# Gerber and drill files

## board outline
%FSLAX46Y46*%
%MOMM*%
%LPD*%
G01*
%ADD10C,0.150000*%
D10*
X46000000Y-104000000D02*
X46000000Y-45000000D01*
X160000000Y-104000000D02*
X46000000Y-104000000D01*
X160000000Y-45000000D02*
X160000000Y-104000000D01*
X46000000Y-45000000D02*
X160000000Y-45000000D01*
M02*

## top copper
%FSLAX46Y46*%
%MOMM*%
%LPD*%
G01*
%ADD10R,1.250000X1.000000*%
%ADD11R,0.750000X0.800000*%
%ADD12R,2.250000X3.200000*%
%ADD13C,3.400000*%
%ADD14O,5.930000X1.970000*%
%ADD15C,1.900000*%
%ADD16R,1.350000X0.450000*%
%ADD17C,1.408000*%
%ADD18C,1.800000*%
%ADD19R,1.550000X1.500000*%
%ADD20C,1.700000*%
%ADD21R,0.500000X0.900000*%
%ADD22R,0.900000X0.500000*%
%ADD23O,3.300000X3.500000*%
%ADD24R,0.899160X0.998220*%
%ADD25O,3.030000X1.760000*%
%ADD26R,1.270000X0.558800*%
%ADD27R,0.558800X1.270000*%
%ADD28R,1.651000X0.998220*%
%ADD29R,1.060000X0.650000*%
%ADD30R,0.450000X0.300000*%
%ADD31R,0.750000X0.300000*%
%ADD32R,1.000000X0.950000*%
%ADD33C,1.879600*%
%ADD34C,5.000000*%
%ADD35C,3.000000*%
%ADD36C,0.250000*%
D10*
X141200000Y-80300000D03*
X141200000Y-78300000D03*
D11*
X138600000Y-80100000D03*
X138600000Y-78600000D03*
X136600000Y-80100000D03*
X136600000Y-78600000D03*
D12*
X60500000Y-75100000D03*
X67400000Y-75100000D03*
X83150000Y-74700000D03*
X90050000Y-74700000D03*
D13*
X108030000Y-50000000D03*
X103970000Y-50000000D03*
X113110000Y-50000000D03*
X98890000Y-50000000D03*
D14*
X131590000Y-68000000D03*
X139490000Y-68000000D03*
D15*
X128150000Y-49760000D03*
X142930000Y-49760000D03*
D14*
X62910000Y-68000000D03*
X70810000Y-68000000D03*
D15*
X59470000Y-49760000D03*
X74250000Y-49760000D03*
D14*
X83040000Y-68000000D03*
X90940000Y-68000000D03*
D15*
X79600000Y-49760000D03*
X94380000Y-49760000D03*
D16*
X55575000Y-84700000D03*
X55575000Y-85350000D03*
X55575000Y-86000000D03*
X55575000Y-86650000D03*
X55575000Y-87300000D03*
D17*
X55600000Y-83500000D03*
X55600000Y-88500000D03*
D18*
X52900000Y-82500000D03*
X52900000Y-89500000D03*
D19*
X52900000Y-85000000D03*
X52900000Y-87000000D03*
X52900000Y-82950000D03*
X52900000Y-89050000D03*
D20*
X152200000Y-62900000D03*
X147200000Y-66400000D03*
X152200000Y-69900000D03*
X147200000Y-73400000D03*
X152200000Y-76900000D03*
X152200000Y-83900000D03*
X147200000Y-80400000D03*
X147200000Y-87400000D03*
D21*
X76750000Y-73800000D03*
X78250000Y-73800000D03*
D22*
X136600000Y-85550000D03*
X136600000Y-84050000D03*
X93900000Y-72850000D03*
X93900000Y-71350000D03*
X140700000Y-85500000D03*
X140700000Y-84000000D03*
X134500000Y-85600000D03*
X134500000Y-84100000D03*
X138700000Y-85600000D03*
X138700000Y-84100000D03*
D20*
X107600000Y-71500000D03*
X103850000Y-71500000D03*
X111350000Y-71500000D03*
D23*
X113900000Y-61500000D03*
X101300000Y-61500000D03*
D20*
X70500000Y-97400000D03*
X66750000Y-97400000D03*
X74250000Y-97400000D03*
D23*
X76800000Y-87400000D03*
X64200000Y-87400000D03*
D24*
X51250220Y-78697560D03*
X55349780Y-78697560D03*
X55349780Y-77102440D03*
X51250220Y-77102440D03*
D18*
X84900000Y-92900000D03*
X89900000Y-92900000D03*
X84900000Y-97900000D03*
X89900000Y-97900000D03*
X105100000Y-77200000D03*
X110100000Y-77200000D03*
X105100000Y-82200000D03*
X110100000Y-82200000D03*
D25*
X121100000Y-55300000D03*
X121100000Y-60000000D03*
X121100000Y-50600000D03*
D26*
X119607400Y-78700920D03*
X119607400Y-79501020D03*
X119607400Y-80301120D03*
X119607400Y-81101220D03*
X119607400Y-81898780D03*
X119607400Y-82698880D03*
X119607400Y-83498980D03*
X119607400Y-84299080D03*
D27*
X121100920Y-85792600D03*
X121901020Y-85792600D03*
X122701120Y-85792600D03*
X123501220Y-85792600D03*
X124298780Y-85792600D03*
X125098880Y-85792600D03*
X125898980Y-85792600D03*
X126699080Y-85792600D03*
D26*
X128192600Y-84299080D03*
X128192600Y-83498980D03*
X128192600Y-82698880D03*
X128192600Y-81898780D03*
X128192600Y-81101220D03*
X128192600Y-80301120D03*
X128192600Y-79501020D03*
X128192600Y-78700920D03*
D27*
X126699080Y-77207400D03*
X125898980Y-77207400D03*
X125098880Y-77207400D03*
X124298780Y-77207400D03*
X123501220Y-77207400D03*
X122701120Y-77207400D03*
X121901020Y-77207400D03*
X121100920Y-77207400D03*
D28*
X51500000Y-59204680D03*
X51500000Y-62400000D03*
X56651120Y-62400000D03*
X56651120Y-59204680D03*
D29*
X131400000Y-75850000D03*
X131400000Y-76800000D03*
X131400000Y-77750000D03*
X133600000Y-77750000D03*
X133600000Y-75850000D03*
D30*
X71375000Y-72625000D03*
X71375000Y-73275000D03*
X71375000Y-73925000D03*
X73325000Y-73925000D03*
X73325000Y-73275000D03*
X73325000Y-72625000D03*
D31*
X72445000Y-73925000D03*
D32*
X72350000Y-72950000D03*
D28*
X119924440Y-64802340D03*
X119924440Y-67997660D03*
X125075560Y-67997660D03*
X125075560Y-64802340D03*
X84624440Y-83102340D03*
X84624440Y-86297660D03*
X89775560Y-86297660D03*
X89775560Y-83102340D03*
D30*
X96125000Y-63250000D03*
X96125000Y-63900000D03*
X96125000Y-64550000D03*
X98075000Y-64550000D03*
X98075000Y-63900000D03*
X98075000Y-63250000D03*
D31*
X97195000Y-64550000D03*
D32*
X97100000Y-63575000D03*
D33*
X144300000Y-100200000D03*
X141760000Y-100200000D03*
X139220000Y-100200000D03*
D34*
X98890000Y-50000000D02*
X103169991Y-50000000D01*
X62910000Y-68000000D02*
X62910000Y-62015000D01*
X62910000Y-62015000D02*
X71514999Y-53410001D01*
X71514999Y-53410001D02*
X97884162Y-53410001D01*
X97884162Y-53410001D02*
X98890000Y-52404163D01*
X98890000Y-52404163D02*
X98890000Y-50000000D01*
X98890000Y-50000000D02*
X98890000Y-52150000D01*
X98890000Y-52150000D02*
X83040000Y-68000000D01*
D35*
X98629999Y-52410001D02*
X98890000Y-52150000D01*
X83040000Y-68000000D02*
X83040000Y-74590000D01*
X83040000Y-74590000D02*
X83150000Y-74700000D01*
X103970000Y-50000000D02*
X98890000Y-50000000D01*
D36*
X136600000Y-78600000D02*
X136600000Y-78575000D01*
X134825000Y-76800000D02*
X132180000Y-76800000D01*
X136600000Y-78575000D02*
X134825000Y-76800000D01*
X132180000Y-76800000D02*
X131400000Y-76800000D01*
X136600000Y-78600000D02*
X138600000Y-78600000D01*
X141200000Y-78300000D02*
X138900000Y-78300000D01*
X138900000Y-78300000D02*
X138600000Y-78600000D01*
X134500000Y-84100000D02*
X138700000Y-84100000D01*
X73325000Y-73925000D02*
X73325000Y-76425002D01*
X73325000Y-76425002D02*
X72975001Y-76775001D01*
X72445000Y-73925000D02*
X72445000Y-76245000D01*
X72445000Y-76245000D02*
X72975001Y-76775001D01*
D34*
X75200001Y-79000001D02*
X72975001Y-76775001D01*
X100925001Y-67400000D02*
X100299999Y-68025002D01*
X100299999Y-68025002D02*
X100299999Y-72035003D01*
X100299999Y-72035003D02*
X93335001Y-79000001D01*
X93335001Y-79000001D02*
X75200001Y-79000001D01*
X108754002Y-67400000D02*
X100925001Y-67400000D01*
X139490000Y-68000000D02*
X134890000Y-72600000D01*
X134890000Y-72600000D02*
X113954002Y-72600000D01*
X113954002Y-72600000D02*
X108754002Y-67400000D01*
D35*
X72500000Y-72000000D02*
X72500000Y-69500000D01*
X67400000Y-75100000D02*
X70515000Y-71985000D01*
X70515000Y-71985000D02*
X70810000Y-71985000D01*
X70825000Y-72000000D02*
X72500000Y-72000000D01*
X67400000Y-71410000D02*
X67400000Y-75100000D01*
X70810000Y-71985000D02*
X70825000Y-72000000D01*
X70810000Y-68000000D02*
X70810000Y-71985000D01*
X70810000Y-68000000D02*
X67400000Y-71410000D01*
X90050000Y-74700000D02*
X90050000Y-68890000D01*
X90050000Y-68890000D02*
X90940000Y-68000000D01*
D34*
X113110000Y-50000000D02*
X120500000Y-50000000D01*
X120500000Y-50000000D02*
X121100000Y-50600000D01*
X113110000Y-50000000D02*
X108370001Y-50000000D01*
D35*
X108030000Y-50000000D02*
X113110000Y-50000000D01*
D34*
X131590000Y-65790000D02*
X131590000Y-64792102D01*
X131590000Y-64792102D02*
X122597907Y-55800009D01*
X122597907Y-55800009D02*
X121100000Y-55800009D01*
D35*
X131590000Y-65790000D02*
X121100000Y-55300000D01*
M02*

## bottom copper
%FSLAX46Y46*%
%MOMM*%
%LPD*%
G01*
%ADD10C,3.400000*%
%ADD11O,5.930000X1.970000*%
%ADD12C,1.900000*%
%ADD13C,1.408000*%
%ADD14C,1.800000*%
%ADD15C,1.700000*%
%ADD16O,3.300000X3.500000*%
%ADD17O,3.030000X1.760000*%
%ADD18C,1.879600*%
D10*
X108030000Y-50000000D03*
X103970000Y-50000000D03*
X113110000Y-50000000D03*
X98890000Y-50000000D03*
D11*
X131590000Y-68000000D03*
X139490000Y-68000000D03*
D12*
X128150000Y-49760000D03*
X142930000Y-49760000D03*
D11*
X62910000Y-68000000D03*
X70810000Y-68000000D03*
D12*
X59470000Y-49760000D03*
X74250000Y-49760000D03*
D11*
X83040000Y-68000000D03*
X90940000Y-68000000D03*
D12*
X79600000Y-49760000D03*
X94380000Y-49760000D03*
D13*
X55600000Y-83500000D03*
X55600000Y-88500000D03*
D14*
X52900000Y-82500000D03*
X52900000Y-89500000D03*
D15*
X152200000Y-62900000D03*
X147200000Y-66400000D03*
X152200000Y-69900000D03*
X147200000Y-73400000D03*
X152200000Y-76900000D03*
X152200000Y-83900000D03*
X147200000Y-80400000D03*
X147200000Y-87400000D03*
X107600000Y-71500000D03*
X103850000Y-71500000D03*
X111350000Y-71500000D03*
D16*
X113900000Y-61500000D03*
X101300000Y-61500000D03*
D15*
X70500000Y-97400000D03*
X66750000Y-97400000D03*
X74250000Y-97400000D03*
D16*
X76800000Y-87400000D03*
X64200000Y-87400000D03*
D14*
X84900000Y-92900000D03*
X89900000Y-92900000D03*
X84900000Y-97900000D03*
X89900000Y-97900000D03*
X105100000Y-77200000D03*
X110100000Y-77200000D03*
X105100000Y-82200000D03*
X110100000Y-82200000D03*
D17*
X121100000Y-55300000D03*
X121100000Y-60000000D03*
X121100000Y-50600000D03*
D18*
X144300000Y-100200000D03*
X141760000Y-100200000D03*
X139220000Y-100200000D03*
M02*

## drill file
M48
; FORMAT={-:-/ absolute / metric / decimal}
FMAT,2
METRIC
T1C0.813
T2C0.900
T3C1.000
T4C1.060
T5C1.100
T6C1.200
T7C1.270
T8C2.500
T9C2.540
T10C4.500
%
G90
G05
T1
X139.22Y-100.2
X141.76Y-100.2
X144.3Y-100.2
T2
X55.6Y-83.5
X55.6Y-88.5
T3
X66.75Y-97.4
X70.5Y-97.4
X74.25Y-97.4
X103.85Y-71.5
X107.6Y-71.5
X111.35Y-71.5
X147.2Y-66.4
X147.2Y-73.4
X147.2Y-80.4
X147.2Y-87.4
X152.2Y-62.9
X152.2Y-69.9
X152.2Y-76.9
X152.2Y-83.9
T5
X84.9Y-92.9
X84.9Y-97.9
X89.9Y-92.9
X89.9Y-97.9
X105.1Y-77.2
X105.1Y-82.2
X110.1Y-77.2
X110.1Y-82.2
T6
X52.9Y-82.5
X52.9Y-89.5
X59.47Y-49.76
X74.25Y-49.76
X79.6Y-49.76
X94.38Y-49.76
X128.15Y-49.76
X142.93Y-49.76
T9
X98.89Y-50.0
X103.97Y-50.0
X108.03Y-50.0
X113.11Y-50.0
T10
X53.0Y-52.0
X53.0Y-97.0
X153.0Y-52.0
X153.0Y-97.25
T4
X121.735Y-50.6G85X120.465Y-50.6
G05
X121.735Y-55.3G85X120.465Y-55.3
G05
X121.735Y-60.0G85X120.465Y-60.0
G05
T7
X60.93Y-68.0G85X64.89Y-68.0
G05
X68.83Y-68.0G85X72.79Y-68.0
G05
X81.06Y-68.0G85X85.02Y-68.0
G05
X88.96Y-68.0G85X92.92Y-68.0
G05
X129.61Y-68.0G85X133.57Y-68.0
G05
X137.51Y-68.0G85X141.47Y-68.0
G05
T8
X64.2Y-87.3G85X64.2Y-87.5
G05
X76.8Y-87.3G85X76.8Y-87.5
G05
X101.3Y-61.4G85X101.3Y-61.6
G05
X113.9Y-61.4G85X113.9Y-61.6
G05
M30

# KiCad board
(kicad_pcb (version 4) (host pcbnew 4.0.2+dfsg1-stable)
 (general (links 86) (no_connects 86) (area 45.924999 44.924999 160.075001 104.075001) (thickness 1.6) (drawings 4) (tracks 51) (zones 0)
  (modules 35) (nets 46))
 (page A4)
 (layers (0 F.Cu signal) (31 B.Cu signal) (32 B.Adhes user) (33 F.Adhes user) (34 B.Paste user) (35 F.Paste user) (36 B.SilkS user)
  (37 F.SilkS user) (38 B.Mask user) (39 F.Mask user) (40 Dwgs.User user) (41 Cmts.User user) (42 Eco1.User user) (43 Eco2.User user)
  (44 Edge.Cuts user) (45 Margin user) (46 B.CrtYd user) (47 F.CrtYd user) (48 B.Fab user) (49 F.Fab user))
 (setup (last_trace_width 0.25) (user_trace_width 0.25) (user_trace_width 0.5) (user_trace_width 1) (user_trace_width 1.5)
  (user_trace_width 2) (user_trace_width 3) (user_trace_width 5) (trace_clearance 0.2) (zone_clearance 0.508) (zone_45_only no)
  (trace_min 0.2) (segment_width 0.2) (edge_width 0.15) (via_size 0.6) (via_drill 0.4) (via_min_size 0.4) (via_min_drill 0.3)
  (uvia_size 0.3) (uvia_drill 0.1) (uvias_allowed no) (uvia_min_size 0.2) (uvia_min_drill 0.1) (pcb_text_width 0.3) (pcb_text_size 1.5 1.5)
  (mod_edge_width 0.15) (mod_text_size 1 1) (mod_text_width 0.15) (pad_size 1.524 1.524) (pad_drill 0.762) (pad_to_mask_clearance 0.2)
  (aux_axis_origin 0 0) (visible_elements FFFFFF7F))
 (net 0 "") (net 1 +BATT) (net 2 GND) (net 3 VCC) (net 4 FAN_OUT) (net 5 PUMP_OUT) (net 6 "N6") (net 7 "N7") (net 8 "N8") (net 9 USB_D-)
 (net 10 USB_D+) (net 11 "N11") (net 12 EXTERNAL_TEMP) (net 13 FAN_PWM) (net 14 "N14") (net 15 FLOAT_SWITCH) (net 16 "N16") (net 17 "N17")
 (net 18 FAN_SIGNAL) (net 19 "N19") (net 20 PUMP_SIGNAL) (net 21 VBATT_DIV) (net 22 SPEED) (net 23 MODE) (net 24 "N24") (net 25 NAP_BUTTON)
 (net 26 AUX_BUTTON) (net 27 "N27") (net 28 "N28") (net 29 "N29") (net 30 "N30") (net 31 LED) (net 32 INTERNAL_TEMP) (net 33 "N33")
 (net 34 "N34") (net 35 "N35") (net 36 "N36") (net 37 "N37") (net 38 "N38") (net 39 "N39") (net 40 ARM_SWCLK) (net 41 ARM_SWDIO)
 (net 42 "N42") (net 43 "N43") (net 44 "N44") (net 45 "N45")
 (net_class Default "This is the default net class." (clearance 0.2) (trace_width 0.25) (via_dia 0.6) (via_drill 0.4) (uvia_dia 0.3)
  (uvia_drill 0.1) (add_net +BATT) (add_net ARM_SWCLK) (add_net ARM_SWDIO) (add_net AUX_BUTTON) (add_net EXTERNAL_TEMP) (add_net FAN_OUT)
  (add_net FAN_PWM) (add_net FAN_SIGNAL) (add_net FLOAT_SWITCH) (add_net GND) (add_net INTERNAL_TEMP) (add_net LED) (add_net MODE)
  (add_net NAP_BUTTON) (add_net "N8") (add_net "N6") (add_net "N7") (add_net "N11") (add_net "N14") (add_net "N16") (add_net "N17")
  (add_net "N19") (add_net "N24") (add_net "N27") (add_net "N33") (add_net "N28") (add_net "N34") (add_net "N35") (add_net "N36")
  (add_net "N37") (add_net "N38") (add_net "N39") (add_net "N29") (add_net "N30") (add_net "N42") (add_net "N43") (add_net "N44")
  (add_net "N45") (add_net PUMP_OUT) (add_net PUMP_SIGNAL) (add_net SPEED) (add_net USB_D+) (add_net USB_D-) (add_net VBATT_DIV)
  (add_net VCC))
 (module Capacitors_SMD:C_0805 (layer F.Cu) (at 141.2 79.3 90)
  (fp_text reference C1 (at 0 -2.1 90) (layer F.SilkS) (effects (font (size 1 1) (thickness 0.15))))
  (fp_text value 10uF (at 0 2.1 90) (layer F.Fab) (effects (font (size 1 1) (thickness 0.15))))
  (pad 1 smd rect (at -1 0 90) (size 1 1.25) (layers F.Cu F.Paste F.Mask) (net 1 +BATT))
  (pad 2 smd rect (at 1 0 90) (size 1 1.25) (layers F.Cu F.Paste F.Mask) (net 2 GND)))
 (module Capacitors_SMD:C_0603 (layer F.Cu) (at 138.6 79.35 90)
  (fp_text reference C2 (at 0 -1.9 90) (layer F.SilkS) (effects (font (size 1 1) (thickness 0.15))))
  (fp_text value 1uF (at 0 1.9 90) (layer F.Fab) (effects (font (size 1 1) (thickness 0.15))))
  (pad 1 smd rect (at -0.75 0 90) (size 0.8 0.75) (layers F.Cu F.Paste F.Mask) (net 1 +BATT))
  (pad 2 smd rect (at 0.75 0 90) (size 0.8 0.75) (layers F.Cu F.Paste F.Mask) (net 2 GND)))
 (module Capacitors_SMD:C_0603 (layer F.Cu) (at 136.6 79.35 90)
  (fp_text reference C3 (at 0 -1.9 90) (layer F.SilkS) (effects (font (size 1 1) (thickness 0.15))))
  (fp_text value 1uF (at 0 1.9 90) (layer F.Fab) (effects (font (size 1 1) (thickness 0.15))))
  (pad 1 smd rect (at -0.75 0 90) (size 0.8 0.75) (layers F.Cu F.Paste F.Mask) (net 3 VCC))
  (pad 2 smd rect (at 0.75 0 90) (size 0.8 0.75) (layers F.Cu F.Paste F.Mask) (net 2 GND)))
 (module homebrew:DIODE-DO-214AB (layer F.Cu) (at 63.95 75.1)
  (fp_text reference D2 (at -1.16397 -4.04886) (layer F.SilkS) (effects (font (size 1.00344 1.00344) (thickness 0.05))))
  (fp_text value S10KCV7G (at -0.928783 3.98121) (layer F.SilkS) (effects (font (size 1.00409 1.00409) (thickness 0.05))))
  (pad 1 smd rect (at -3.45 0) (size 2.25 3.2) (layers F.Cu F.Paste F.Mask) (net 1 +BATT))
  (pad 2 smd rect (at 3.45 0) (size 2.25 3.2) (layers F.Cu F.Paste F.Mask) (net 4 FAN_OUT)))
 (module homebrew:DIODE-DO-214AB (layer F.Cu) (at 86.6 74.7)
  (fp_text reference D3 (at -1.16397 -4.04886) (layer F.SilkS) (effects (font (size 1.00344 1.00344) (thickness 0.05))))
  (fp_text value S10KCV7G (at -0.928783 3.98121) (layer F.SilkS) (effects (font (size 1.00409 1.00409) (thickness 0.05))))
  (pad 1 smd rect (at -3.45 0) (size 2.25 3.2) (layers F.Cu F.Paste F.Mask) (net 1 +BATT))
  (pad 2 smd rect (at 3.45 0) (size 2.25 3.2) (layers F.Cu F.Paste F.Mask) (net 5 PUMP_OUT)))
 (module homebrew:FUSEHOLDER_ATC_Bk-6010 (layer F.Cu) (at 106 50 180)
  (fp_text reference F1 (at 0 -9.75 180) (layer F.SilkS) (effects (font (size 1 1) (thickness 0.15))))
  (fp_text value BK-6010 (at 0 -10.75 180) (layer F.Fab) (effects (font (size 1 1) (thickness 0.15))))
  (pad 1 thru_hole circle (at -2.03 0 180) (size 3.4 3.4) (drill 2.54) (layers *.Cu *.Mask) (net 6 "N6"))
  (pad 2 thru_hole circle (at 2.03 0 180) (size 3.4 3.4) (drill 2.54) (layers *.Cu *.Mask) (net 1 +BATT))
  (pad 1 thru_hole circle (at -7.11 0 180) (size 3.4 3.4) (drill 2.54) (layers *.Cu *.Mask) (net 6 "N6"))
  (pad 2 thru_hole circle (at 7.11 0 180) (size 3.4 3.4) (drill 2.54) (layers *.Cu *.Mask) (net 1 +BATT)))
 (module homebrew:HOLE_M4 (layer F.Cu) (at 153 52)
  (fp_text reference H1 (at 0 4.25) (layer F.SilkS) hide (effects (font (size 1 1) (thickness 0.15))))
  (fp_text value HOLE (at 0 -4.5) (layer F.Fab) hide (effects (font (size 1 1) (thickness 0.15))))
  (pad "" np_thru_hole circle (at 0 0) (size 4.5 4.5) (drill 4.5) (layers *.Cu *.Mask) (clearance 2.2)))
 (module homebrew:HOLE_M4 (layer F.Cu) (at 53 52)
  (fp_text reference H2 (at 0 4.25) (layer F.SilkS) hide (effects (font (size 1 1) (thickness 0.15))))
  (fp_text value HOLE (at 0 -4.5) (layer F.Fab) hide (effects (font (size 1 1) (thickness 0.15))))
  (pad "" np_thru_hole circle (at 0 0) (size 4.5 4.5) (drill 4.5) (layers *.Cu *.Mask) (clearance 2.2)))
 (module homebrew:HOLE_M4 (layer F.Cu) (at 53 97)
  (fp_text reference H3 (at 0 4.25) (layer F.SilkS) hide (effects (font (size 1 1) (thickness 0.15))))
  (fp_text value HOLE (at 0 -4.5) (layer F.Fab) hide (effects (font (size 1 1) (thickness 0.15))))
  (pad "" np_thru_hole circle (at 0 0) (size 4.5 4.5) (drill 4.5) (layers *.Cu *.Mask) (clearance 2.2)))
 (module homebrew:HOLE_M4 (layer F.Cu) (at 153 97.25)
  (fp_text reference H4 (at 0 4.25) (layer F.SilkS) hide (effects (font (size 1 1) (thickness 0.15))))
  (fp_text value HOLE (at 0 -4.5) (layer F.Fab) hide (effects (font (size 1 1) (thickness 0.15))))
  (pad "" np_thru_hole circle (at 0 0) (size 4.5 4.5) (drill 4.5) (layers *.Cu *.Mask) (clearance 2.2)))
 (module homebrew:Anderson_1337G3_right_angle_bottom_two (layer F.Cu) (at 135.54 68)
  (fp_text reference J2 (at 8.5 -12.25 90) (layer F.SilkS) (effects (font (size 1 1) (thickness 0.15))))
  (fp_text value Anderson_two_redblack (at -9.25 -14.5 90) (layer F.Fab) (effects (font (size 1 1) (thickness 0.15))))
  (pad 1 thru_hole oval (at -3.95 0) (size 5.93 1.97) (drill oval 5.23 1.27) (layers *.Cu *.Mask) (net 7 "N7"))
  (pad 2 thru_hole oval (at 3.95 0) (size 5.93 1.97) (drill oval 5.23 1.27) (layers *.Cu *.Mask) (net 2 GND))
  (pad "" thru_hole circle (at -7.39 -18.24) (size 1.9 1.9) (drill 1.2) (layers *.Cu *.Mask))
  (pad "" thru_hole circle (at 7.39 -18.24) (size 1.9 1.9) (drill 1.2) (layers *.Cu *.Mask)))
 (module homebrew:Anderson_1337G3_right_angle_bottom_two (layer F.Cu) (at 66.86 68)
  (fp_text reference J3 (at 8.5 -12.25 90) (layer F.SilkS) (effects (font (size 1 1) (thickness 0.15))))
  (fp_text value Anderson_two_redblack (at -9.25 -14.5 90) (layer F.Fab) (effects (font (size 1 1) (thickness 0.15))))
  (pad 1 thru_hole oval (at -3.95 0) (size 5.93 1.97) (drill oval 5.23 1.27) (layers *.Cu *.Mask) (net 1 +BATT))
  (pad 2 thru_hole oval (at 3.95 0) (size 5.93 1.97) (drill oval 5.23 1.27) (layers *.Cu *.Mask) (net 4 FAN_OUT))
  (pad "" thru_hole circle (at -7.39 -18.24) (size 1.9 1.9) (drill 1.2) (layers *.Cu *.Mask))
  (pad "" thru_hole circle (at 7.39 -18.24) (size 1.9 1.9) (drill 1.2) (layers *.Cu *.Mask)))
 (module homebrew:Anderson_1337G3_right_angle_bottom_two (layer F.Cu) (at 86.99 68)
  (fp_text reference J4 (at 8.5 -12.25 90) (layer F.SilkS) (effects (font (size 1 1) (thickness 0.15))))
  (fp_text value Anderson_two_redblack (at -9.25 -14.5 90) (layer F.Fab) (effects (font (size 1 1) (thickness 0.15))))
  (pad 1 thru_hole oval (at -3.95 0) (size 5.93 1.97) (drill oval 5.23 1.27) (layers *.Cu *.Mask) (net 1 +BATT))
  (pad 2 thru_hole oval (at 3.95 0) (size 5.93 1.97) (drill oval 5.23 1.27) (layers *.Cu *.Mask) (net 5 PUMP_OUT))
  (pad "" thru_hole circle (at -7.39 -18.24) (size 1.9 1.9) (drill 1.2) (layers *.Cu *.Mask))
  (pad "" thru_hole circle (at 7.39 -18.24) (size 1.9 1.9) (drill 1.2) (layers *.Cu *.Mask)))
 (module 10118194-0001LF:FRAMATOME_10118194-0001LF (layer F.Cu) (at 52.9 86 270)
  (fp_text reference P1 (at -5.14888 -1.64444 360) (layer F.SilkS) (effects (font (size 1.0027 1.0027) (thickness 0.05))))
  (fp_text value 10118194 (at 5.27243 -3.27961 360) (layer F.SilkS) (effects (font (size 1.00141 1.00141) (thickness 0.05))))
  (pad 1 smd rect (at -1.3 -2.675 90) (size 0.45 1.35) (layers F.Cu F.Paste F.Mask) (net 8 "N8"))
  (pad 2 smd rect (at -0.65 -2.675 90) (size 0.45 1.35) (layers F.Cu F.Paste F.Mask) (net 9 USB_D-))
  (pad 3 smd rect (at 0 -2.675 90) (size 0.45 1.35) (layers F.Cu F.Paste F.Mask) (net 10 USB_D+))
  (pad 4 smd rect (at 0.65 -2.675 90) (size 0.45 1.35) (layers F.Cu F.Paste F.Mask) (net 2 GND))
  (pad 5 smd rect (at 1.3 -2.675 90) (size 0.45 1.35) (layers F.Cu F.Paste F.Mask) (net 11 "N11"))
  (pad P$6 thru_hole circle (at -2.5 -2.7 270) (size 1.408 1.408) (drill 0.9) (layers *.Cu *.Mask F.SilkS))
  (pad P$7 thru_hole circle (at 2.5 -2.7 270) (size 1.408 1.408) (drill 0.9) (layers *.Cu *.Mask F.SilkS))
  (pad P$8 thru_hole circle (at -3.5 0 270) (size 1.8 1.8) (drill 1.2) (layers *.Cu *.Mask F.SilkS))
  (pad P$9 thru_hole circle (at 3.5 0 270) (size 1.8 1.8) (drill 1.2) (layers *.Cu *.Mask F.SilkS))
  (pad P$10 smd rect (at -1 0 270) (size 1.5 1.55) (layers F.Cu F.Paste F.Mask))
  (pad P$11 smd rect (at 1 0 270) (size 1.5 1.55) (layers F.Cu F.Paste F.Mask))
  (pad P$12 smd rect (at -3.05 0 270) (size 1.5 1.55) (layers F.Cu F.Paste F.Mask))
  (pad P$13 smd rect (at 3.05 0 270) (size 1.5 1.55) (layers F.Cu F.Paste F.Mask)))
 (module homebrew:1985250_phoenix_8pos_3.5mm (layer F.Cu) (at 152.2 62.9 90)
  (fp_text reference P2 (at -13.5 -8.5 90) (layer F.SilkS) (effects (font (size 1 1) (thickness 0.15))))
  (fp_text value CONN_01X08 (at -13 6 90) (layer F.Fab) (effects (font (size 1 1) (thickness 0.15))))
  (pad 1 thru_hole circle (at 0 0 90) (size 1.7 1.7) (drill 1) (layers *.Cu *.Mask) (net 3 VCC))
  (pad 2 thru_hole circle (at -3.5 -5 90) (size 1.7 1.7) (drill 1) (layers *.Cu *.Mask) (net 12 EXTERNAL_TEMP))
  (pad 3 thru_hole circle (at -7 0 90) (size 1.7 1.7) (drill 1) (layers *.Cu *.Mask) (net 2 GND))
  (pad 4 thru_hole circle (at -10.5 -5 90) (size 1.7 1.7) (drill 1) (layers *.Cu *.Mask) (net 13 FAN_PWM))
  (pad 5 thru_hole circle (at -14 0 90) (size 1.7 1.7) (drill 1) (layers *.Cu *.Mask) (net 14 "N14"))
  (pad 7 thru_hole circle (at -21 0 90) (size 1.7 1.7) (drill 1) (layers *.Cu *.Mask) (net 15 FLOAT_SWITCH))
  (pad 6 thru_hole circle (at -17.5 -5 90) (size 1.7 1.7) (drill 1) (layers *.Cu *.Mask) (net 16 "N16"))
  (pad 8 thru_hole circle (at -24.5 -5 90) (size 1.7 1.7) (drill 1) (layers *.Cu *.Mask) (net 2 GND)))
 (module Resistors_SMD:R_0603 (layer F.Cu) (at 77.5 73.8)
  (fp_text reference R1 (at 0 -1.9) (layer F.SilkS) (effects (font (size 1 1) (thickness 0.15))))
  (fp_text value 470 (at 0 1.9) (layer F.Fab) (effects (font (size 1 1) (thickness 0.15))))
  (pad 1 smd rect (at -0.75 0) (size 0.5 0.9) (layers F.Cu F.Paste F.Mask) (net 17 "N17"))
  (pad 2 smd rect (at 0.75 0) (size 0.5 0.9) (layers F.Cu F.Paste F.Mask) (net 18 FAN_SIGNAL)))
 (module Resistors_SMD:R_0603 (layer F.Cu) (at 136.6 84.8 90)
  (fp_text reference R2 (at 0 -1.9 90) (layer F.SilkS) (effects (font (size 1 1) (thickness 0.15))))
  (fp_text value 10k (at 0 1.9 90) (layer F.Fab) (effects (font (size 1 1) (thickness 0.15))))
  (pad 1 smd rect (at -0.75 0 90) (size 0.5 0.9) (layers F.Cu F.Paste F.Mask) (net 17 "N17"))
  (pad 2 smd rect (at 0.75 0 90) (size 0.5 0.9) (layers F.Cu F.Paste F.Mask) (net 2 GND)))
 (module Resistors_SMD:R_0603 (layer F.Cu) (at 93.9 72.1 90)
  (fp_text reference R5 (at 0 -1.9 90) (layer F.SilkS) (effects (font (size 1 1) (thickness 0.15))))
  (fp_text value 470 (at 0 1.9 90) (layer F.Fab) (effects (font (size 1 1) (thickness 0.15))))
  (pad 1 smd rect (at -0.75 0 90) (size 0.5 0.9) (layers F.Cu F.Paste F.Mask) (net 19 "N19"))
  (pad 2 smd rect (at 0.75 0 90) (size 0.5 0.9) (layers F.Cu F.Paste F.Mask) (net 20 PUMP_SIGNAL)))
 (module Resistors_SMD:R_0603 (layer F.Cu) (at 140.7 84.75 90)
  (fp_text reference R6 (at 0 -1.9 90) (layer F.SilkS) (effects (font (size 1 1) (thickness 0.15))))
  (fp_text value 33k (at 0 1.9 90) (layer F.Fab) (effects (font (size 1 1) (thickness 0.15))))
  (pad 1 smd rect (at -0.75 0 90) (size 0.5 0.9) (layers F.Cu F.Paste F.Mask) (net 1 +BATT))
  (pad 2 smd rect (at 0.75 0 90) (size 0.5 0.9) (layers F.Cu F.Paste F.Mask) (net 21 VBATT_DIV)))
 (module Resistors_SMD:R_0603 (layer F.Cu) (at 134.5 84.85 90)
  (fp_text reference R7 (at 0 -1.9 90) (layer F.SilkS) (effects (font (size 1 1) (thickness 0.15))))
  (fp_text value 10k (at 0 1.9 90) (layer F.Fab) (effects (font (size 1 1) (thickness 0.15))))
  (pad 1 smd rect (at -0.75 0 90) (size 0.5 0.9) (layers F.Cu F.Paste F.Mask) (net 21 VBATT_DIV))
  (pad 2 smd rect (at 0.75 0 90) (size 0.5 0.9) (layers F.Cu F.Paste F.Mask) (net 2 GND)))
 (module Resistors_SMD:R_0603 (layer F.Cu) (at 138.7 84.85 90)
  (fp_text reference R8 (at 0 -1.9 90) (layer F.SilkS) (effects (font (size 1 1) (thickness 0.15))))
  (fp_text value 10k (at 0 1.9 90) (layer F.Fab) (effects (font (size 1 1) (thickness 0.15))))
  (pad 1 smd rect (at -0.75 0 90) (size 0.5 0.9) (layers F.Cu F.Paste F.Mask) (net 19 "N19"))
  (pad 2 smd rect (at 0.75 0 90) (size 0.5 0.9) (layers F.Cu F.Paste F.Mask) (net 2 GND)))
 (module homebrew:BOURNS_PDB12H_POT (layer F.Cu) (at 107.6 71.5)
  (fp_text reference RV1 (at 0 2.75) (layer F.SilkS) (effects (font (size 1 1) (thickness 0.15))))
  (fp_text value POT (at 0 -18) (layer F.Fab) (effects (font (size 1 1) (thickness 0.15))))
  (pad 2 thru_hole circle (at 0 0) (size 1.7 1.7) (drill 1) (layers *.Cu *.Mask) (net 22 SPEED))
  (pad 1 thru_hole circle (at -3.75 0) (size 1.7 1.7) (drill 1) (layers *.Cu *.Mask) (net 3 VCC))
  (pad 3 thru_hole circle (at 3.75 0) (size 1.7 1.7) (drill 1) (layers *.Cu *.Mask) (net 2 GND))
  (pad "" thru_hole oval (at 6.3 -10) (size 3.3 3.5) (drill oval 2.5 2.7) (layers *.Cu *.Mask))
  (pad "" thru_hole oval (at -6.3 -10) (size 3.3 3.5) (drill oval 2.5 2.7) (layers *.Cu *.Mask)))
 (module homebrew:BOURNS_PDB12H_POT (layer F.Cu) (at 70.5 97.4)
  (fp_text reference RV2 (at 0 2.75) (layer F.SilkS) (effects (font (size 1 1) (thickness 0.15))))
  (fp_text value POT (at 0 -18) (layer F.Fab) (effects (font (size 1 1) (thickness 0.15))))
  (pad 2 thru_hole circle (at 0 0) (size 1.7 1.7) (drill 1) (layers *.Cu *.Mask) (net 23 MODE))
  (pad 1 thru_hole circle (at -3.75 0) (size 1.7 1.7) (drill 1) (layers *.Cu *.Mask) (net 3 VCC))
  (pad 3 thru_hole circle (at 3.75 0) (size 1.7 1.7) (drill 1) (layers *.Cu *.Mask) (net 2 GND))
  (pad "" thru_hole oval (at 6.3 -10) (size 3.3 3.5) (drill oval 2.5 2.7) (layers *.Cu *.Mask))
  (pad "" thru_hole oval (at -6.3 -10) (size 3.3 3.5) (drill oval 2.5 2.7) (layers *.Cu *.Mask)))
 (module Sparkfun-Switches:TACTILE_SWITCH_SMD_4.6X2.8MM (layer F.Cu) (at 53.3 77.9)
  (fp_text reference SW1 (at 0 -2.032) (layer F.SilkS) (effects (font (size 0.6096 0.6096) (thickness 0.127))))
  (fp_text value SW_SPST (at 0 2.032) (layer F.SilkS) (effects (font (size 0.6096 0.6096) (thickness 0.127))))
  (pad 1 smd rect (at -2.04978 0.79756) (size 0.89916 0.99822) (layers F.Cu F.Paste F.Mask) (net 2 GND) (solder_mask_margin 0.1016))
  (pad 2 smd rect (at 2.04978 0.79756) (size 0.89916 0.99822) (layers F.Cu F.Paste F.Mask) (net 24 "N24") (solder_mask_margin 0.1016))
  (pad 3 smd rect (at 2.04978 -0.79756) (size 0.89916 0.99822) (layers F.Cu F.Paste F.Mask) (solder_mask_margin 0.1016))
  (pad 4 smd rect (at -2.04978 -0.79756) (size 0.89916 0.99822) (layers F.Cu F.Paste F.Mask) (solder_mask_margin 0.1016)))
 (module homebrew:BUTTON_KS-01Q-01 (layer F.Cu) (at 84.9 92.9)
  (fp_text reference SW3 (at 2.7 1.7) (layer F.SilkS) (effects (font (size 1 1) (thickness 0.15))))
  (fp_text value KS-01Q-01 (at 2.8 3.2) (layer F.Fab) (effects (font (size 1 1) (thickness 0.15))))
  (pad 1 thru_hole circle (at 0 0) (size 1.8 1.8) (drill 1.1) (layers *.Cu *.Mask F.SilkS) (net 2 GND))
  (pad 2 thru_hole circle (at 5 0) (size 1.8 1.8) (drill 1.1) (layers *.Cu *.Mask F.SilkS) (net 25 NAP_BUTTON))
  (pad 1 thru_hole circle (at 0 5) (size 1.8 1.8) (drill 1.1) (layers *.Cu *.Mask F.SilkS) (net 2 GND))
  (pad 2 thru_hole circle (at 5 5) (size 1.8 1.8) (drill 1.1) (layers *.Cu *.Mask F.SilkS) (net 25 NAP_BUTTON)))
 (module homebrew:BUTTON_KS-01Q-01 (layer F.Cu) (at 105.1 77.2)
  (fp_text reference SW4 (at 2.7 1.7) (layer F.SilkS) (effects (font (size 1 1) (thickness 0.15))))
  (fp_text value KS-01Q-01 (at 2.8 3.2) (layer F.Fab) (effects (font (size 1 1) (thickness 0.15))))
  (pad 1 thru_hole circle (at 0 0) (size 1.8 1.8) (drill 1.1) (layers *.Cu *.Mask F.SilkS) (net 2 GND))
  (pad 2 thru_hole circle (at 5 0) (size 1.8 1.8) (drill 1.1) (layers *.Cu *.Mask F.SilkS) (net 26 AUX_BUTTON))
  (pad 1 thru_hole circle (at 0 5) (size 1.8 1.8) (drill 1.1) (layers *.Cu *.Mask F.SilkS) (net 2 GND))
  (pad 2 thru_hole circle (at 5 5) (size 1.8 1.8) (drill 1.1) (layers *.Cu *.Mask F.SilkS) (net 26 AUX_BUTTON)))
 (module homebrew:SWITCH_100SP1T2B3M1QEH (layer F.Cu) (at 121.1 55.3 270)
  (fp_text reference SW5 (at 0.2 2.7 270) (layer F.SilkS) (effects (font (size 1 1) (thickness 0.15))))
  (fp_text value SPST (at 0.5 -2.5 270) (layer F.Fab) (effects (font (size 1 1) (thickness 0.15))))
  (pad 2 thru_hole oval (at 0 0 270) (size 1.76 3.03) (drill oval 1.06 2.33) (layers *.Cu *.Mask F.SilkS) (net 7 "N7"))
  (pad 3 thru_hole oval (at 4.7 0 270) (size 1.76 3.03) (drill oval 1.06 2.33) (layers *.Cu *.Mask F.SilkS))
  (pad 1 thru_hole oval (at -4.7 0 270) (size 1.76 3.03) (drill oval 1.06 2.33) (layers *.Cu *.Mask F.SilkS) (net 6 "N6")))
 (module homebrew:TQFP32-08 (layer F.Cu) (at 123.9 81.5)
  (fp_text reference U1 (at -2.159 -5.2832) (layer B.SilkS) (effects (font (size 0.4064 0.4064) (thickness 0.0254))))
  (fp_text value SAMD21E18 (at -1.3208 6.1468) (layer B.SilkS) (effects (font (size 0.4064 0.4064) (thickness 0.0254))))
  (pad 1 smd rect (at -4.2926 -2.79908) (size 1.27 0.5588) (layers F.Cu F.Paste F.Mask) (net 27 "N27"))
  (pad 2 smd rect (at -4.2926 -1.99898) (size 1.27 0.5588) (layers F.Cu F.Paste F.Mask) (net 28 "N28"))
  (pad 3 smd rect (at -4.2926 -1.19888) (size 1.27 0.5588) (layers F.Cu F.Paste F.Mask) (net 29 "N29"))
  (pad 4 smd rect (at -4.2926 -0.39878) (size 1.27 0.5588) (layers F.Cu F.Paste F.Mask) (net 21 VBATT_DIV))
  (pad 5 smd rect (at -4.2926 0.39878) (size 1.27 0.5588) (layers F.Cu F.Paste F.Mask) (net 23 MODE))
  (pad 6 smd rect (at -4.2926 1.19888) (size 1.27 0.5588) (layers F.Cu F.Paste F.Mask) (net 22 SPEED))
  (pad 7 smd rect (at -4.2926 1.99898) (size 1.27 0.5588) (layers F.Cu F.Paste F.Mask) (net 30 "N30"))
  (pad 8 smd rect (at -4.2926 2.79908) (size 1.27 0.5588) (layers F.Cu F.Paste F.Mask) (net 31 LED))
  (pad 9 smd rect (at -2.79908 4.2926) (size 0.5588 1.27) (layers F.Cu F.Paste F.Mask) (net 3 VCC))
  (pad 10 smd rect (at -1.99898 4.2926) (size 0.5588 1.27) (layers F.Cu F.Paste F.Mask) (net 2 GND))
  (pad 11 smd rect (at -1.19888 4.2926) (size 0.5588 1.27) (layers F.Cu F.Paste F.Mask) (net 18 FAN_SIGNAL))
  (pad 12 smd rect (at -0.39878 4.2926) (size 0.5588 1.27) (layers F.Cu F.Paste F.Mask) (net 20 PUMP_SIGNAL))
  (pad 13 smd rect (at 0.39878 4.2926) (size 0.5588 1.27) (layers F.Cu F.Paste F.Mask) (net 13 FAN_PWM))
  (pad 14 smd rect (at 1.19888 4.2926) (size 0.5588 1.27) (layers F.Cu F.Paste F.Mask) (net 25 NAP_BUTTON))
  (pad 15 smd rect (at 1.99898 4.2926) (size 0.5588 1.27) (layers F.Cu F.Paste F.Mask) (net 26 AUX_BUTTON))
  (pad 16 smd rect (at 2.79908 4.2926) (size 0.5588 1.27) (layers F.Cu F.Paste F.Mask) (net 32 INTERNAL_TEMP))
  (pad 17 smd rect (at 4.2926 2.79908) (size 1.27 0.5588) (layers F.Cu F.Paste F.Mask) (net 12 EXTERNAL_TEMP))
  (pad 18 smd rect (at 4.2926 1.99898) (size 1.27 0.5588) (layers F.Cu F.Paste F.Mask) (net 15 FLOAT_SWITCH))
  (pad 19 smd rect (at 4.2926 1.19888) (size 1.27 0.5588) (layers F.Cu F.Paste F.Mask) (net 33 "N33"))
  (pad 20 smd rect (at 4.2926 0.39878) (size 1.27 0.5588) (layers F.Cu F.Paste F.Mask) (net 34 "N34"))
  (pad 21 smd rect (at 4.2926 -0.39878) (size 1.27 0.5588) (layers F.Cu F.Paste F.Mask) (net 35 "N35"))
  (pad 22 smd rect (at 4.2926 -1.19888) (size 1.27 0.5588) (layers F.Cu F.Paste F.Mask) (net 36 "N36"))
  (pad 23 smd rect (at 4.2926 -1.99898) (size 1.27 0.5588) (layers F.Cu F.Paste F.Mask) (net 9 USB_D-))
  (pad 24 smd rect (at 4.2926 -2.79908) (size 1.27 0.5588) (layers F.Cu F.Paste F.Mask) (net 10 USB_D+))
  (pad 25 smd rect (at 2.79908 -4.2926) (size 0.5588 1.27) (layers F.Cu F.Paste F.Mask) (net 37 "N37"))
  (pad 26 smd rect (at 1.99898 -4.2926) (size 0.5588 1.27) (layers F.Cu F.Paste F.Mask) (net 24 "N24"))
  (pad 27 smd rect (at 1.19888 -4.2926) (size 0.5588 1.27) (layers F.Cu F.Paste F.Mask) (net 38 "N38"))
  (pad 28 smd rect (at 0.39878 -4.2926) (size 0.5588 1.27) (layers F.Cu F.Paste F.Mask) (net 2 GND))
  (pad 29 smd rect (at -0.39878 -4.2926) (size 0.5588 1.27) (layers F.Cu F.Paste F.Mask) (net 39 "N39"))
  (pad 30 smd rect (at -1.19888 -4.2926) (size 0.5588 1.27) (layers F.Cu F.Paste F.Mask) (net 3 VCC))
  (pad 31 smd rect (at -1.99898 -4.2926) (size 0.5588 1.27) (layers F.Cu F.Paste F.Mask) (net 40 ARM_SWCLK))
  (pad 32 smd rect (at -2.79908 -4.2926) (size 0.5588 1.27) (layers F.Cu F.Paste F.Mask) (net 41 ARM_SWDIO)))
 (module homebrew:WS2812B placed (layer F.Cu) (at 54.07556 60.80234)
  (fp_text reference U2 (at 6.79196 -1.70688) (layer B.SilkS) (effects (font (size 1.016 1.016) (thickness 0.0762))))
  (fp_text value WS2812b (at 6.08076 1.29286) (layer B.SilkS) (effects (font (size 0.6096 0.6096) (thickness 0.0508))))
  (pad 1 smd rect (at -2.57556 -1.59766) (size 1.651 0.99822) (layers F.Cu F.Paste F.Mask) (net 3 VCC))
  (pad 2 smd rect (at -2.57556 1.59766) (size 1.651 0.99822) (layers F.Cu F.Paste F.Mask) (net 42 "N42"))
  (pad 3 smd rect (at 2.57556 1.59766) (size 1.651 0.99822) (layers F.Cu F.Paste F.Mask) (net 2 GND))
  (pad 4 smd rect (at 2.57556 -1.59766) (size 1.651 0.99822) (layers F.Cu F.Paste F.Mask) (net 31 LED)))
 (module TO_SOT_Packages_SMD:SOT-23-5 (layer F.Cu) (at 132.5 76.8)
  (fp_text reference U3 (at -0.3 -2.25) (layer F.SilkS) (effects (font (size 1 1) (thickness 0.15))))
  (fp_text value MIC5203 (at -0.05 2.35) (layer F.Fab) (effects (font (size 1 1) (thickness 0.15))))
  (pad 1 smd rect (at -1.1 -0.95) (size 1.06 0.65) (layers F.Cu F.Paste F.Mask) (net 1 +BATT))
  (pad 2 smd rect (at -1.1 0) (size 1.06 0.65) (layers F.Cu F.Paste F.Mask) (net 2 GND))
  (pad 3 smd rect (at -1.1 0.95) (size 1.06 0.65) (layers F.Cu F.Paste F.Mask) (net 1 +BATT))
  (pad 4 smd rect (at 1.1 0.95) (size 1.06 0.65) (layers F.Cu F.Paste F.Mask) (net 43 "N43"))
  (pad 5 smd rect (at 1.1 -0.95) (size 1.06 0.65) (layers F.Cu F.Paste F.Mask) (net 3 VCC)))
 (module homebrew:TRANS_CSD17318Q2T (layer F.Cu) (at 72.35 73.275)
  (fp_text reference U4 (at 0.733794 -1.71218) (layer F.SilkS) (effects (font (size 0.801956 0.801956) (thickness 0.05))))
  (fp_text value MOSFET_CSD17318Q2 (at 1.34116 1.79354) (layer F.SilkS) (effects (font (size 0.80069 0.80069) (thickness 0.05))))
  (pad 3 smd rect (at -0.975 -0.65) (size 0.45 0.3) (layers F.Cu F.Paste F.Mask) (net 4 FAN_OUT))
  (pad 3 smd rect (at -0.975 0) (size 0.45 0.3) (layers F.Cu F.Paste F.Mask) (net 4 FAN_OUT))
  (pad 2 smd rect (at -0.975 0.65) (size 0.45 0.3) (layers F.Cu F.Paste F.Mask) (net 17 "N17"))
  (pad 1 smd rect (at 0.975 0.65 180) (size 0.45 0.3) (layers F.Cu F.Paste F.Mask) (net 2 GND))
  (pad 3 smd rect (at 0.975 0 180) (size 0.45 0.3) (layers F.Cu F.Paste F.Mask) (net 4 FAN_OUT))
  (pad 3 smd rect (at 0.975 -0.65 180) (size 0.45 0.3) (layers F.Cu F.Paste F.Mask) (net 4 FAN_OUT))
  (pad 1 smd rect (at 0.095 0.65) (size 0.75 0.3) (layers F.Cu F.Paste F.Mask) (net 2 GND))
  (pad 3 smd rect (at 0 -0.325) (size 1 0.95) (layers F.Cu F.Paste F.Mask) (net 4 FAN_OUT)))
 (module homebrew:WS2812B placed (layer F.Cu) (at 122.5 66.4)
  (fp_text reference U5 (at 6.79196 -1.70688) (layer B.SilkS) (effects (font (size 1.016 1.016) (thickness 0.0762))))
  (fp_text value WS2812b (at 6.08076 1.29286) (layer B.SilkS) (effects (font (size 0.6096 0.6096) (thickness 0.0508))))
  (pad 1 smd rect (at -2.57556 -1.59766) (size 1.651 0.99822) (layers F.Cu F.Paste F.Mask) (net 3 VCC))
  (pad 2 smd rect (at -2.57556 1.59766) (size 1.651 0.99822) (layers F.Cu F.Paste F.Mask) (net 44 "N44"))
  (pad 3 smd rect (at 2.57556 1.59766) (size 1.651 0.99822) (layers F.Cu F.Paste F.Mask) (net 2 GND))
  (pad 4 smd rect (at 2.57556 -1.59766) (size 1.651 0.99822) (layers F.Cu F.Paste F.Mask) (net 42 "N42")))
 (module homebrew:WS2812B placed (layer F.Cu) (at 87.2 84.7)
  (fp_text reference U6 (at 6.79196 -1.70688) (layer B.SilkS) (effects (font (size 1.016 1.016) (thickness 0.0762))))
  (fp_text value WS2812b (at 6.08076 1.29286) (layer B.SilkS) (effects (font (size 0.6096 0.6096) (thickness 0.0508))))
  (pad 1 smd rect (at -2.57556 -1.59766) (size 1.651 0.99822) (layers F.Cu F.Paste F.Mask) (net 3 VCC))
  (pad 2 smd rect (at -2.57556 1.59766) (size 1.651 0.99822) (layers F.Cu F.Paste F.Mask) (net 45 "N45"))
  (pad 3 smd rect (at 2.57556 1.59766) (size 1.651 0.99822) (layers F.Cu F.Paste F.Mask) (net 2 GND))
  (pad 4 smd rect (at 2.57556 -1.59766) (size 1.651 0.99822) (layers F.Cu F.Paste F.Mask) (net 44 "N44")))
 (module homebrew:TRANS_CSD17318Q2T (layer F.Cu) (at 97.1 63.9)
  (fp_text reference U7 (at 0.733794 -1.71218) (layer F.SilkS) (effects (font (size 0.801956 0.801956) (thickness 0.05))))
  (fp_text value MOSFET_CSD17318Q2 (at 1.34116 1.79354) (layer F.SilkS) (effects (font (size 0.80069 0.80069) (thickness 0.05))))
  (pad 3 smd rect (at -0.975 -0.65) (size 0.45 0.3) (layers F.Cu F.Paste F.Mask) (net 5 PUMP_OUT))
  (pad 3 smd rect (at -0.975 0) (size 0.45 0.3) (layers F.Cu F.Paste F.Mask) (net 5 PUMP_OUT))
  (pad 2 smd rect (at -0.975 0.65) (size 0.45 0.3) (layers F.Cu F.Paste F.Mask) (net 19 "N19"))
  (pad 1 smd rect (at 0.975 0.65 180) (size 0.45 0.3) (layers F.Cu F.Paste F.Mask) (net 2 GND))
  (pad 3 smd rect (at 0.975 0 180) (size 0.45 0.3) (layers F.Cu F.Paste F.Mask) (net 5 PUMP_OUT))
  (pad 3 smd rect (at 0.975 -0.65 180) (size 0.45 0.3) (layers F.Cu F.Paste F.Mask) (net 5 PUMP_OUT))
  (pad 1 smd rect (at 0.095 0.65) (size 0.75 0.3) (layers F.Cu F.Paste F.Mask) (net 2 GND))
  (pad 3 smd rect (at 0 -0.325) (size 1 0.95) (layers F.Cu F.Paste F.Mask) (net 5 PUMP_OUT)))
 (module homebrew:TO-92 (layer F.Cu) (at 141.76 100.2)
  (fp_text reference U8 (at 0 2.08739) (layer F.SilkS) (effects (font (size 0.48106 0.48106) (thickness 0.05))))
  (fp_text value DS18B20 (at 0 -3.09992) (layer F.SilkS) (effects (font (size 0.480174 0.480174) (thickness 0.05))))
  (pad 3 thru_hole circle (at 2.54 0) (size 1.8796 1.8796) (drill 0.8128) (layers *.Cu *.Mask) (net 3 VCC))
  (pad 2 thru_hole circle (at 0 0) (size 1.8796 1.8796) (drill 0.8128) (layers *.Cu *.Mask) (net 32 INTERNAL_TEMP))
  (pad 1 thru_hole circle (at -2.54 0) (size 1.8796 1.8796) (drill 0.8128) (layers *.Cu *.Mask) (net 2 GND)))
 (gr_line (start 46 104) (end 46 45) (layer Edge.Cuts) (width 0.15))
 (gr_line (start 160 104) (end 46 104) (layer Edge.Cuts) (width 0.15))
 (gr_line (start 160 45) (end 160 104) (layer Edge.Cuts) (width 0.15))
 (gr_line (start 46 45) (end 160 45) (layer Edge.Cuts) (width 0.15))
 (segment (start 98.89 50) (end 103.169991 50) (width 5) (layer F.Cu) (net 1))
 (segment (start 62.91 68) (end 62.91 62.015) (width 5) (layer F.Cu) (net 1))
 (segment (start 62.91 62.015) (end 71.514999 53.410001) (width 5) (layer F.Cu) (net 1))
 (segment (start 71.514999 53.410001) (end 97.884162 53.410001) (width 5) (layer F.Cu) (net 1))
 (segment (start 97.884162 53.410001) (end 98.89 52.404163) (width 5) (layer F.Cu) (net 1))
 (segment (start 98.89 52.404163) (end 98.89 50) (width 5) (layer F.Cu) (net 1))
 (segment (start 98.89 50) (end 98.89 52.15) (width 5) (layer F.Cu) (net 1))
 (segment (start 98.89 52.15) (end 83.04 68) (width 5) (layer F.Cu) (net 1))
 (segment (start 98.629999 52.410001) (end 98.89 52.15) (width 3) (layer F.Cu) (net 1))
 (segment (start 83.04 68) (end 83.04 74.59) (width 3) (layer F.Cu) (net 1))
 (segment (start 83.04 74.59) (end 83.15 74.7) (width 3) (layer F.Cu) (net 1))
 (segment (start 103.97 50) (end 98.89 50) (width 3) (layer F.Cu) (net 1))
 (segment (start 136.6 78.6) (end 136.6 78.575) (width 0.25) (layer F.Cu) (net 2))
 (segment (start 134.825 76.8) (end 132.18 76.8) (width 0.25) (layer F.Cu) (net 2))
 (segment (start 136.6 78.575) (end 134.825 76.8) (width 0.25) (layer F.Cu) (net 2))
 (segment (start 132.18 76.8) (end 131.4 76.8) (width 0.25) (layer F.Cu) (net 2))
 (segment (start 136.6 78.6) (end 138.6 78.6) (width 0.25) (layer F.Cu) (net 2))
 (segment (start 141.2 78.3) (end 138.9 78.3) (width 0.25) (layer F.Cu) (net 2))
 (segment (start 138.9 78.3) (end 138.6 78.6) (width 0.25) (layer F.Cu) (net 2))
 (segment (start 134.5 84.1) (end 138.7 84.1) (width 0.25) (layer F.Cu) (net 2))
 (segment (start 73.325 73.925) (end 73.325 76.425002) (width 0.25) (layer F.Cu) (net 2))
 (segment (start 73.325 76.425002) (end 72.975001 76.775001) (width 0.25) (layer F.Cu) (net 2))
 (segment (start 72.445 73.925) (end 72.445 76.245) (width 0.25) (layer F.Cu) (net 2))
 (segment (start 72.445 76.245) (end 72.975001 76.775001) (width 0.25) (layer F.Cu) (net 2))
 (segment (start 75.200001 79.000001) (end 72.975001 76.775001) (width 5) (layer F.Cu) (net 2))
 (segment (start 100.925001 67.4) (end 100.299999 68.025002) (width 5) (layer F.Cu) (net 2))
 (segment (start 100.299999 68.025002) (end 100.299999 72.035003) (width 5) (layer F.Cu) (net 2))
 (segment (start 100.299999 72.035003) (end 93.335001 79.000001) (width 5) (layer F.Cu) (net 2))
 (segment (start 93.335001 79.000001) (end 75.200001 79.000001) (width 5) (layer F.Cu) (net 2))
 (segment (start 108.754002 67.4) (end 100.925001 67.4) (width 5) (layer F.Cu) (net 2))
 (segment (start 139.49 68) (end 134.89 72.6) (width 5) (layer F.Cu) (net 2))
 (segment (start 134.89 72.6) (end 113.954002 72.6) (width 5) (layer F.Cu) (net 2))
 (segment (start 113.954002 72.6) (end 108.754002 67.4) (width 5) (layer F.Cu) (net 2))
 (segment (start 72.5 72) (end 72.5 69.5) (width 3) (layer F.Cu) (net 4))
 (segment (start 67.4 75.1) (end 70.515 71.985) (width 3) (layer F.Cu) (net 4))
 (segment (start 70.515 71.985) (end 70.81 71.985) (width 3) (layer F.Cu) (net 4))
 (segment (start 70.825 72) (end 72.5 72) (width 3) (layer F.Cu) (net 4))
 (segment (start 67.4 71.41) (end 67.4 75.1) (width 3) (layer F.Cu) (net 4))
 (segment (start 70.81 71.985) (end 70.825 72) (width 3) (layer F.Cu) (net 4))
 (segment (start 70.81 68) (end 70.81 71.985) (width 3) (layer F.Cu) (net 4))
 (segment (start 70.81 68) (end 67.4 71.41) (width 3) (layer F.Cu) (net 4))
 (segment (start 90.05 74.7) (end 90.05 68.89) (width 3) (layer F.Cu) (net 5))
 (segment (start 90.05 68.89) (end 90.94 68) (width 3) (layer F.Cu) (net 5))
 (segment (start 113.11 50) (end 120.5 50) (width 5) (layer F.Cu) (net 6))
 (segment (start 120.5 50) (end 121.1 50.6) (width 5) (layer F.Cu) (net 6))
 (segment (start 113.11 50) (end 108.370001 50) (width 5) (layer F.Cu) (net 6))
 (segment (start 108.03 50) (end 113.11 50) (width 3) (layer F.Cu) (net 6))
 (segment (start 131.59 65.79) (end 131.59 64.792102) (width 5) (layer F.Cu) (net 7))
 (segment (start 131.59 64.792102) (end 122.597907 55.800009) (width 5) (layer F.Cu) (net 7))
 (segment (start 122.597907 55.800009) (end 121.1 55.800009) (width 5) (layer F.Cu) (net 7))
 (segment (start 131.59 65.79) (end 121.1 55.3) (width 3) (layer F.Cu) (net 7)))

